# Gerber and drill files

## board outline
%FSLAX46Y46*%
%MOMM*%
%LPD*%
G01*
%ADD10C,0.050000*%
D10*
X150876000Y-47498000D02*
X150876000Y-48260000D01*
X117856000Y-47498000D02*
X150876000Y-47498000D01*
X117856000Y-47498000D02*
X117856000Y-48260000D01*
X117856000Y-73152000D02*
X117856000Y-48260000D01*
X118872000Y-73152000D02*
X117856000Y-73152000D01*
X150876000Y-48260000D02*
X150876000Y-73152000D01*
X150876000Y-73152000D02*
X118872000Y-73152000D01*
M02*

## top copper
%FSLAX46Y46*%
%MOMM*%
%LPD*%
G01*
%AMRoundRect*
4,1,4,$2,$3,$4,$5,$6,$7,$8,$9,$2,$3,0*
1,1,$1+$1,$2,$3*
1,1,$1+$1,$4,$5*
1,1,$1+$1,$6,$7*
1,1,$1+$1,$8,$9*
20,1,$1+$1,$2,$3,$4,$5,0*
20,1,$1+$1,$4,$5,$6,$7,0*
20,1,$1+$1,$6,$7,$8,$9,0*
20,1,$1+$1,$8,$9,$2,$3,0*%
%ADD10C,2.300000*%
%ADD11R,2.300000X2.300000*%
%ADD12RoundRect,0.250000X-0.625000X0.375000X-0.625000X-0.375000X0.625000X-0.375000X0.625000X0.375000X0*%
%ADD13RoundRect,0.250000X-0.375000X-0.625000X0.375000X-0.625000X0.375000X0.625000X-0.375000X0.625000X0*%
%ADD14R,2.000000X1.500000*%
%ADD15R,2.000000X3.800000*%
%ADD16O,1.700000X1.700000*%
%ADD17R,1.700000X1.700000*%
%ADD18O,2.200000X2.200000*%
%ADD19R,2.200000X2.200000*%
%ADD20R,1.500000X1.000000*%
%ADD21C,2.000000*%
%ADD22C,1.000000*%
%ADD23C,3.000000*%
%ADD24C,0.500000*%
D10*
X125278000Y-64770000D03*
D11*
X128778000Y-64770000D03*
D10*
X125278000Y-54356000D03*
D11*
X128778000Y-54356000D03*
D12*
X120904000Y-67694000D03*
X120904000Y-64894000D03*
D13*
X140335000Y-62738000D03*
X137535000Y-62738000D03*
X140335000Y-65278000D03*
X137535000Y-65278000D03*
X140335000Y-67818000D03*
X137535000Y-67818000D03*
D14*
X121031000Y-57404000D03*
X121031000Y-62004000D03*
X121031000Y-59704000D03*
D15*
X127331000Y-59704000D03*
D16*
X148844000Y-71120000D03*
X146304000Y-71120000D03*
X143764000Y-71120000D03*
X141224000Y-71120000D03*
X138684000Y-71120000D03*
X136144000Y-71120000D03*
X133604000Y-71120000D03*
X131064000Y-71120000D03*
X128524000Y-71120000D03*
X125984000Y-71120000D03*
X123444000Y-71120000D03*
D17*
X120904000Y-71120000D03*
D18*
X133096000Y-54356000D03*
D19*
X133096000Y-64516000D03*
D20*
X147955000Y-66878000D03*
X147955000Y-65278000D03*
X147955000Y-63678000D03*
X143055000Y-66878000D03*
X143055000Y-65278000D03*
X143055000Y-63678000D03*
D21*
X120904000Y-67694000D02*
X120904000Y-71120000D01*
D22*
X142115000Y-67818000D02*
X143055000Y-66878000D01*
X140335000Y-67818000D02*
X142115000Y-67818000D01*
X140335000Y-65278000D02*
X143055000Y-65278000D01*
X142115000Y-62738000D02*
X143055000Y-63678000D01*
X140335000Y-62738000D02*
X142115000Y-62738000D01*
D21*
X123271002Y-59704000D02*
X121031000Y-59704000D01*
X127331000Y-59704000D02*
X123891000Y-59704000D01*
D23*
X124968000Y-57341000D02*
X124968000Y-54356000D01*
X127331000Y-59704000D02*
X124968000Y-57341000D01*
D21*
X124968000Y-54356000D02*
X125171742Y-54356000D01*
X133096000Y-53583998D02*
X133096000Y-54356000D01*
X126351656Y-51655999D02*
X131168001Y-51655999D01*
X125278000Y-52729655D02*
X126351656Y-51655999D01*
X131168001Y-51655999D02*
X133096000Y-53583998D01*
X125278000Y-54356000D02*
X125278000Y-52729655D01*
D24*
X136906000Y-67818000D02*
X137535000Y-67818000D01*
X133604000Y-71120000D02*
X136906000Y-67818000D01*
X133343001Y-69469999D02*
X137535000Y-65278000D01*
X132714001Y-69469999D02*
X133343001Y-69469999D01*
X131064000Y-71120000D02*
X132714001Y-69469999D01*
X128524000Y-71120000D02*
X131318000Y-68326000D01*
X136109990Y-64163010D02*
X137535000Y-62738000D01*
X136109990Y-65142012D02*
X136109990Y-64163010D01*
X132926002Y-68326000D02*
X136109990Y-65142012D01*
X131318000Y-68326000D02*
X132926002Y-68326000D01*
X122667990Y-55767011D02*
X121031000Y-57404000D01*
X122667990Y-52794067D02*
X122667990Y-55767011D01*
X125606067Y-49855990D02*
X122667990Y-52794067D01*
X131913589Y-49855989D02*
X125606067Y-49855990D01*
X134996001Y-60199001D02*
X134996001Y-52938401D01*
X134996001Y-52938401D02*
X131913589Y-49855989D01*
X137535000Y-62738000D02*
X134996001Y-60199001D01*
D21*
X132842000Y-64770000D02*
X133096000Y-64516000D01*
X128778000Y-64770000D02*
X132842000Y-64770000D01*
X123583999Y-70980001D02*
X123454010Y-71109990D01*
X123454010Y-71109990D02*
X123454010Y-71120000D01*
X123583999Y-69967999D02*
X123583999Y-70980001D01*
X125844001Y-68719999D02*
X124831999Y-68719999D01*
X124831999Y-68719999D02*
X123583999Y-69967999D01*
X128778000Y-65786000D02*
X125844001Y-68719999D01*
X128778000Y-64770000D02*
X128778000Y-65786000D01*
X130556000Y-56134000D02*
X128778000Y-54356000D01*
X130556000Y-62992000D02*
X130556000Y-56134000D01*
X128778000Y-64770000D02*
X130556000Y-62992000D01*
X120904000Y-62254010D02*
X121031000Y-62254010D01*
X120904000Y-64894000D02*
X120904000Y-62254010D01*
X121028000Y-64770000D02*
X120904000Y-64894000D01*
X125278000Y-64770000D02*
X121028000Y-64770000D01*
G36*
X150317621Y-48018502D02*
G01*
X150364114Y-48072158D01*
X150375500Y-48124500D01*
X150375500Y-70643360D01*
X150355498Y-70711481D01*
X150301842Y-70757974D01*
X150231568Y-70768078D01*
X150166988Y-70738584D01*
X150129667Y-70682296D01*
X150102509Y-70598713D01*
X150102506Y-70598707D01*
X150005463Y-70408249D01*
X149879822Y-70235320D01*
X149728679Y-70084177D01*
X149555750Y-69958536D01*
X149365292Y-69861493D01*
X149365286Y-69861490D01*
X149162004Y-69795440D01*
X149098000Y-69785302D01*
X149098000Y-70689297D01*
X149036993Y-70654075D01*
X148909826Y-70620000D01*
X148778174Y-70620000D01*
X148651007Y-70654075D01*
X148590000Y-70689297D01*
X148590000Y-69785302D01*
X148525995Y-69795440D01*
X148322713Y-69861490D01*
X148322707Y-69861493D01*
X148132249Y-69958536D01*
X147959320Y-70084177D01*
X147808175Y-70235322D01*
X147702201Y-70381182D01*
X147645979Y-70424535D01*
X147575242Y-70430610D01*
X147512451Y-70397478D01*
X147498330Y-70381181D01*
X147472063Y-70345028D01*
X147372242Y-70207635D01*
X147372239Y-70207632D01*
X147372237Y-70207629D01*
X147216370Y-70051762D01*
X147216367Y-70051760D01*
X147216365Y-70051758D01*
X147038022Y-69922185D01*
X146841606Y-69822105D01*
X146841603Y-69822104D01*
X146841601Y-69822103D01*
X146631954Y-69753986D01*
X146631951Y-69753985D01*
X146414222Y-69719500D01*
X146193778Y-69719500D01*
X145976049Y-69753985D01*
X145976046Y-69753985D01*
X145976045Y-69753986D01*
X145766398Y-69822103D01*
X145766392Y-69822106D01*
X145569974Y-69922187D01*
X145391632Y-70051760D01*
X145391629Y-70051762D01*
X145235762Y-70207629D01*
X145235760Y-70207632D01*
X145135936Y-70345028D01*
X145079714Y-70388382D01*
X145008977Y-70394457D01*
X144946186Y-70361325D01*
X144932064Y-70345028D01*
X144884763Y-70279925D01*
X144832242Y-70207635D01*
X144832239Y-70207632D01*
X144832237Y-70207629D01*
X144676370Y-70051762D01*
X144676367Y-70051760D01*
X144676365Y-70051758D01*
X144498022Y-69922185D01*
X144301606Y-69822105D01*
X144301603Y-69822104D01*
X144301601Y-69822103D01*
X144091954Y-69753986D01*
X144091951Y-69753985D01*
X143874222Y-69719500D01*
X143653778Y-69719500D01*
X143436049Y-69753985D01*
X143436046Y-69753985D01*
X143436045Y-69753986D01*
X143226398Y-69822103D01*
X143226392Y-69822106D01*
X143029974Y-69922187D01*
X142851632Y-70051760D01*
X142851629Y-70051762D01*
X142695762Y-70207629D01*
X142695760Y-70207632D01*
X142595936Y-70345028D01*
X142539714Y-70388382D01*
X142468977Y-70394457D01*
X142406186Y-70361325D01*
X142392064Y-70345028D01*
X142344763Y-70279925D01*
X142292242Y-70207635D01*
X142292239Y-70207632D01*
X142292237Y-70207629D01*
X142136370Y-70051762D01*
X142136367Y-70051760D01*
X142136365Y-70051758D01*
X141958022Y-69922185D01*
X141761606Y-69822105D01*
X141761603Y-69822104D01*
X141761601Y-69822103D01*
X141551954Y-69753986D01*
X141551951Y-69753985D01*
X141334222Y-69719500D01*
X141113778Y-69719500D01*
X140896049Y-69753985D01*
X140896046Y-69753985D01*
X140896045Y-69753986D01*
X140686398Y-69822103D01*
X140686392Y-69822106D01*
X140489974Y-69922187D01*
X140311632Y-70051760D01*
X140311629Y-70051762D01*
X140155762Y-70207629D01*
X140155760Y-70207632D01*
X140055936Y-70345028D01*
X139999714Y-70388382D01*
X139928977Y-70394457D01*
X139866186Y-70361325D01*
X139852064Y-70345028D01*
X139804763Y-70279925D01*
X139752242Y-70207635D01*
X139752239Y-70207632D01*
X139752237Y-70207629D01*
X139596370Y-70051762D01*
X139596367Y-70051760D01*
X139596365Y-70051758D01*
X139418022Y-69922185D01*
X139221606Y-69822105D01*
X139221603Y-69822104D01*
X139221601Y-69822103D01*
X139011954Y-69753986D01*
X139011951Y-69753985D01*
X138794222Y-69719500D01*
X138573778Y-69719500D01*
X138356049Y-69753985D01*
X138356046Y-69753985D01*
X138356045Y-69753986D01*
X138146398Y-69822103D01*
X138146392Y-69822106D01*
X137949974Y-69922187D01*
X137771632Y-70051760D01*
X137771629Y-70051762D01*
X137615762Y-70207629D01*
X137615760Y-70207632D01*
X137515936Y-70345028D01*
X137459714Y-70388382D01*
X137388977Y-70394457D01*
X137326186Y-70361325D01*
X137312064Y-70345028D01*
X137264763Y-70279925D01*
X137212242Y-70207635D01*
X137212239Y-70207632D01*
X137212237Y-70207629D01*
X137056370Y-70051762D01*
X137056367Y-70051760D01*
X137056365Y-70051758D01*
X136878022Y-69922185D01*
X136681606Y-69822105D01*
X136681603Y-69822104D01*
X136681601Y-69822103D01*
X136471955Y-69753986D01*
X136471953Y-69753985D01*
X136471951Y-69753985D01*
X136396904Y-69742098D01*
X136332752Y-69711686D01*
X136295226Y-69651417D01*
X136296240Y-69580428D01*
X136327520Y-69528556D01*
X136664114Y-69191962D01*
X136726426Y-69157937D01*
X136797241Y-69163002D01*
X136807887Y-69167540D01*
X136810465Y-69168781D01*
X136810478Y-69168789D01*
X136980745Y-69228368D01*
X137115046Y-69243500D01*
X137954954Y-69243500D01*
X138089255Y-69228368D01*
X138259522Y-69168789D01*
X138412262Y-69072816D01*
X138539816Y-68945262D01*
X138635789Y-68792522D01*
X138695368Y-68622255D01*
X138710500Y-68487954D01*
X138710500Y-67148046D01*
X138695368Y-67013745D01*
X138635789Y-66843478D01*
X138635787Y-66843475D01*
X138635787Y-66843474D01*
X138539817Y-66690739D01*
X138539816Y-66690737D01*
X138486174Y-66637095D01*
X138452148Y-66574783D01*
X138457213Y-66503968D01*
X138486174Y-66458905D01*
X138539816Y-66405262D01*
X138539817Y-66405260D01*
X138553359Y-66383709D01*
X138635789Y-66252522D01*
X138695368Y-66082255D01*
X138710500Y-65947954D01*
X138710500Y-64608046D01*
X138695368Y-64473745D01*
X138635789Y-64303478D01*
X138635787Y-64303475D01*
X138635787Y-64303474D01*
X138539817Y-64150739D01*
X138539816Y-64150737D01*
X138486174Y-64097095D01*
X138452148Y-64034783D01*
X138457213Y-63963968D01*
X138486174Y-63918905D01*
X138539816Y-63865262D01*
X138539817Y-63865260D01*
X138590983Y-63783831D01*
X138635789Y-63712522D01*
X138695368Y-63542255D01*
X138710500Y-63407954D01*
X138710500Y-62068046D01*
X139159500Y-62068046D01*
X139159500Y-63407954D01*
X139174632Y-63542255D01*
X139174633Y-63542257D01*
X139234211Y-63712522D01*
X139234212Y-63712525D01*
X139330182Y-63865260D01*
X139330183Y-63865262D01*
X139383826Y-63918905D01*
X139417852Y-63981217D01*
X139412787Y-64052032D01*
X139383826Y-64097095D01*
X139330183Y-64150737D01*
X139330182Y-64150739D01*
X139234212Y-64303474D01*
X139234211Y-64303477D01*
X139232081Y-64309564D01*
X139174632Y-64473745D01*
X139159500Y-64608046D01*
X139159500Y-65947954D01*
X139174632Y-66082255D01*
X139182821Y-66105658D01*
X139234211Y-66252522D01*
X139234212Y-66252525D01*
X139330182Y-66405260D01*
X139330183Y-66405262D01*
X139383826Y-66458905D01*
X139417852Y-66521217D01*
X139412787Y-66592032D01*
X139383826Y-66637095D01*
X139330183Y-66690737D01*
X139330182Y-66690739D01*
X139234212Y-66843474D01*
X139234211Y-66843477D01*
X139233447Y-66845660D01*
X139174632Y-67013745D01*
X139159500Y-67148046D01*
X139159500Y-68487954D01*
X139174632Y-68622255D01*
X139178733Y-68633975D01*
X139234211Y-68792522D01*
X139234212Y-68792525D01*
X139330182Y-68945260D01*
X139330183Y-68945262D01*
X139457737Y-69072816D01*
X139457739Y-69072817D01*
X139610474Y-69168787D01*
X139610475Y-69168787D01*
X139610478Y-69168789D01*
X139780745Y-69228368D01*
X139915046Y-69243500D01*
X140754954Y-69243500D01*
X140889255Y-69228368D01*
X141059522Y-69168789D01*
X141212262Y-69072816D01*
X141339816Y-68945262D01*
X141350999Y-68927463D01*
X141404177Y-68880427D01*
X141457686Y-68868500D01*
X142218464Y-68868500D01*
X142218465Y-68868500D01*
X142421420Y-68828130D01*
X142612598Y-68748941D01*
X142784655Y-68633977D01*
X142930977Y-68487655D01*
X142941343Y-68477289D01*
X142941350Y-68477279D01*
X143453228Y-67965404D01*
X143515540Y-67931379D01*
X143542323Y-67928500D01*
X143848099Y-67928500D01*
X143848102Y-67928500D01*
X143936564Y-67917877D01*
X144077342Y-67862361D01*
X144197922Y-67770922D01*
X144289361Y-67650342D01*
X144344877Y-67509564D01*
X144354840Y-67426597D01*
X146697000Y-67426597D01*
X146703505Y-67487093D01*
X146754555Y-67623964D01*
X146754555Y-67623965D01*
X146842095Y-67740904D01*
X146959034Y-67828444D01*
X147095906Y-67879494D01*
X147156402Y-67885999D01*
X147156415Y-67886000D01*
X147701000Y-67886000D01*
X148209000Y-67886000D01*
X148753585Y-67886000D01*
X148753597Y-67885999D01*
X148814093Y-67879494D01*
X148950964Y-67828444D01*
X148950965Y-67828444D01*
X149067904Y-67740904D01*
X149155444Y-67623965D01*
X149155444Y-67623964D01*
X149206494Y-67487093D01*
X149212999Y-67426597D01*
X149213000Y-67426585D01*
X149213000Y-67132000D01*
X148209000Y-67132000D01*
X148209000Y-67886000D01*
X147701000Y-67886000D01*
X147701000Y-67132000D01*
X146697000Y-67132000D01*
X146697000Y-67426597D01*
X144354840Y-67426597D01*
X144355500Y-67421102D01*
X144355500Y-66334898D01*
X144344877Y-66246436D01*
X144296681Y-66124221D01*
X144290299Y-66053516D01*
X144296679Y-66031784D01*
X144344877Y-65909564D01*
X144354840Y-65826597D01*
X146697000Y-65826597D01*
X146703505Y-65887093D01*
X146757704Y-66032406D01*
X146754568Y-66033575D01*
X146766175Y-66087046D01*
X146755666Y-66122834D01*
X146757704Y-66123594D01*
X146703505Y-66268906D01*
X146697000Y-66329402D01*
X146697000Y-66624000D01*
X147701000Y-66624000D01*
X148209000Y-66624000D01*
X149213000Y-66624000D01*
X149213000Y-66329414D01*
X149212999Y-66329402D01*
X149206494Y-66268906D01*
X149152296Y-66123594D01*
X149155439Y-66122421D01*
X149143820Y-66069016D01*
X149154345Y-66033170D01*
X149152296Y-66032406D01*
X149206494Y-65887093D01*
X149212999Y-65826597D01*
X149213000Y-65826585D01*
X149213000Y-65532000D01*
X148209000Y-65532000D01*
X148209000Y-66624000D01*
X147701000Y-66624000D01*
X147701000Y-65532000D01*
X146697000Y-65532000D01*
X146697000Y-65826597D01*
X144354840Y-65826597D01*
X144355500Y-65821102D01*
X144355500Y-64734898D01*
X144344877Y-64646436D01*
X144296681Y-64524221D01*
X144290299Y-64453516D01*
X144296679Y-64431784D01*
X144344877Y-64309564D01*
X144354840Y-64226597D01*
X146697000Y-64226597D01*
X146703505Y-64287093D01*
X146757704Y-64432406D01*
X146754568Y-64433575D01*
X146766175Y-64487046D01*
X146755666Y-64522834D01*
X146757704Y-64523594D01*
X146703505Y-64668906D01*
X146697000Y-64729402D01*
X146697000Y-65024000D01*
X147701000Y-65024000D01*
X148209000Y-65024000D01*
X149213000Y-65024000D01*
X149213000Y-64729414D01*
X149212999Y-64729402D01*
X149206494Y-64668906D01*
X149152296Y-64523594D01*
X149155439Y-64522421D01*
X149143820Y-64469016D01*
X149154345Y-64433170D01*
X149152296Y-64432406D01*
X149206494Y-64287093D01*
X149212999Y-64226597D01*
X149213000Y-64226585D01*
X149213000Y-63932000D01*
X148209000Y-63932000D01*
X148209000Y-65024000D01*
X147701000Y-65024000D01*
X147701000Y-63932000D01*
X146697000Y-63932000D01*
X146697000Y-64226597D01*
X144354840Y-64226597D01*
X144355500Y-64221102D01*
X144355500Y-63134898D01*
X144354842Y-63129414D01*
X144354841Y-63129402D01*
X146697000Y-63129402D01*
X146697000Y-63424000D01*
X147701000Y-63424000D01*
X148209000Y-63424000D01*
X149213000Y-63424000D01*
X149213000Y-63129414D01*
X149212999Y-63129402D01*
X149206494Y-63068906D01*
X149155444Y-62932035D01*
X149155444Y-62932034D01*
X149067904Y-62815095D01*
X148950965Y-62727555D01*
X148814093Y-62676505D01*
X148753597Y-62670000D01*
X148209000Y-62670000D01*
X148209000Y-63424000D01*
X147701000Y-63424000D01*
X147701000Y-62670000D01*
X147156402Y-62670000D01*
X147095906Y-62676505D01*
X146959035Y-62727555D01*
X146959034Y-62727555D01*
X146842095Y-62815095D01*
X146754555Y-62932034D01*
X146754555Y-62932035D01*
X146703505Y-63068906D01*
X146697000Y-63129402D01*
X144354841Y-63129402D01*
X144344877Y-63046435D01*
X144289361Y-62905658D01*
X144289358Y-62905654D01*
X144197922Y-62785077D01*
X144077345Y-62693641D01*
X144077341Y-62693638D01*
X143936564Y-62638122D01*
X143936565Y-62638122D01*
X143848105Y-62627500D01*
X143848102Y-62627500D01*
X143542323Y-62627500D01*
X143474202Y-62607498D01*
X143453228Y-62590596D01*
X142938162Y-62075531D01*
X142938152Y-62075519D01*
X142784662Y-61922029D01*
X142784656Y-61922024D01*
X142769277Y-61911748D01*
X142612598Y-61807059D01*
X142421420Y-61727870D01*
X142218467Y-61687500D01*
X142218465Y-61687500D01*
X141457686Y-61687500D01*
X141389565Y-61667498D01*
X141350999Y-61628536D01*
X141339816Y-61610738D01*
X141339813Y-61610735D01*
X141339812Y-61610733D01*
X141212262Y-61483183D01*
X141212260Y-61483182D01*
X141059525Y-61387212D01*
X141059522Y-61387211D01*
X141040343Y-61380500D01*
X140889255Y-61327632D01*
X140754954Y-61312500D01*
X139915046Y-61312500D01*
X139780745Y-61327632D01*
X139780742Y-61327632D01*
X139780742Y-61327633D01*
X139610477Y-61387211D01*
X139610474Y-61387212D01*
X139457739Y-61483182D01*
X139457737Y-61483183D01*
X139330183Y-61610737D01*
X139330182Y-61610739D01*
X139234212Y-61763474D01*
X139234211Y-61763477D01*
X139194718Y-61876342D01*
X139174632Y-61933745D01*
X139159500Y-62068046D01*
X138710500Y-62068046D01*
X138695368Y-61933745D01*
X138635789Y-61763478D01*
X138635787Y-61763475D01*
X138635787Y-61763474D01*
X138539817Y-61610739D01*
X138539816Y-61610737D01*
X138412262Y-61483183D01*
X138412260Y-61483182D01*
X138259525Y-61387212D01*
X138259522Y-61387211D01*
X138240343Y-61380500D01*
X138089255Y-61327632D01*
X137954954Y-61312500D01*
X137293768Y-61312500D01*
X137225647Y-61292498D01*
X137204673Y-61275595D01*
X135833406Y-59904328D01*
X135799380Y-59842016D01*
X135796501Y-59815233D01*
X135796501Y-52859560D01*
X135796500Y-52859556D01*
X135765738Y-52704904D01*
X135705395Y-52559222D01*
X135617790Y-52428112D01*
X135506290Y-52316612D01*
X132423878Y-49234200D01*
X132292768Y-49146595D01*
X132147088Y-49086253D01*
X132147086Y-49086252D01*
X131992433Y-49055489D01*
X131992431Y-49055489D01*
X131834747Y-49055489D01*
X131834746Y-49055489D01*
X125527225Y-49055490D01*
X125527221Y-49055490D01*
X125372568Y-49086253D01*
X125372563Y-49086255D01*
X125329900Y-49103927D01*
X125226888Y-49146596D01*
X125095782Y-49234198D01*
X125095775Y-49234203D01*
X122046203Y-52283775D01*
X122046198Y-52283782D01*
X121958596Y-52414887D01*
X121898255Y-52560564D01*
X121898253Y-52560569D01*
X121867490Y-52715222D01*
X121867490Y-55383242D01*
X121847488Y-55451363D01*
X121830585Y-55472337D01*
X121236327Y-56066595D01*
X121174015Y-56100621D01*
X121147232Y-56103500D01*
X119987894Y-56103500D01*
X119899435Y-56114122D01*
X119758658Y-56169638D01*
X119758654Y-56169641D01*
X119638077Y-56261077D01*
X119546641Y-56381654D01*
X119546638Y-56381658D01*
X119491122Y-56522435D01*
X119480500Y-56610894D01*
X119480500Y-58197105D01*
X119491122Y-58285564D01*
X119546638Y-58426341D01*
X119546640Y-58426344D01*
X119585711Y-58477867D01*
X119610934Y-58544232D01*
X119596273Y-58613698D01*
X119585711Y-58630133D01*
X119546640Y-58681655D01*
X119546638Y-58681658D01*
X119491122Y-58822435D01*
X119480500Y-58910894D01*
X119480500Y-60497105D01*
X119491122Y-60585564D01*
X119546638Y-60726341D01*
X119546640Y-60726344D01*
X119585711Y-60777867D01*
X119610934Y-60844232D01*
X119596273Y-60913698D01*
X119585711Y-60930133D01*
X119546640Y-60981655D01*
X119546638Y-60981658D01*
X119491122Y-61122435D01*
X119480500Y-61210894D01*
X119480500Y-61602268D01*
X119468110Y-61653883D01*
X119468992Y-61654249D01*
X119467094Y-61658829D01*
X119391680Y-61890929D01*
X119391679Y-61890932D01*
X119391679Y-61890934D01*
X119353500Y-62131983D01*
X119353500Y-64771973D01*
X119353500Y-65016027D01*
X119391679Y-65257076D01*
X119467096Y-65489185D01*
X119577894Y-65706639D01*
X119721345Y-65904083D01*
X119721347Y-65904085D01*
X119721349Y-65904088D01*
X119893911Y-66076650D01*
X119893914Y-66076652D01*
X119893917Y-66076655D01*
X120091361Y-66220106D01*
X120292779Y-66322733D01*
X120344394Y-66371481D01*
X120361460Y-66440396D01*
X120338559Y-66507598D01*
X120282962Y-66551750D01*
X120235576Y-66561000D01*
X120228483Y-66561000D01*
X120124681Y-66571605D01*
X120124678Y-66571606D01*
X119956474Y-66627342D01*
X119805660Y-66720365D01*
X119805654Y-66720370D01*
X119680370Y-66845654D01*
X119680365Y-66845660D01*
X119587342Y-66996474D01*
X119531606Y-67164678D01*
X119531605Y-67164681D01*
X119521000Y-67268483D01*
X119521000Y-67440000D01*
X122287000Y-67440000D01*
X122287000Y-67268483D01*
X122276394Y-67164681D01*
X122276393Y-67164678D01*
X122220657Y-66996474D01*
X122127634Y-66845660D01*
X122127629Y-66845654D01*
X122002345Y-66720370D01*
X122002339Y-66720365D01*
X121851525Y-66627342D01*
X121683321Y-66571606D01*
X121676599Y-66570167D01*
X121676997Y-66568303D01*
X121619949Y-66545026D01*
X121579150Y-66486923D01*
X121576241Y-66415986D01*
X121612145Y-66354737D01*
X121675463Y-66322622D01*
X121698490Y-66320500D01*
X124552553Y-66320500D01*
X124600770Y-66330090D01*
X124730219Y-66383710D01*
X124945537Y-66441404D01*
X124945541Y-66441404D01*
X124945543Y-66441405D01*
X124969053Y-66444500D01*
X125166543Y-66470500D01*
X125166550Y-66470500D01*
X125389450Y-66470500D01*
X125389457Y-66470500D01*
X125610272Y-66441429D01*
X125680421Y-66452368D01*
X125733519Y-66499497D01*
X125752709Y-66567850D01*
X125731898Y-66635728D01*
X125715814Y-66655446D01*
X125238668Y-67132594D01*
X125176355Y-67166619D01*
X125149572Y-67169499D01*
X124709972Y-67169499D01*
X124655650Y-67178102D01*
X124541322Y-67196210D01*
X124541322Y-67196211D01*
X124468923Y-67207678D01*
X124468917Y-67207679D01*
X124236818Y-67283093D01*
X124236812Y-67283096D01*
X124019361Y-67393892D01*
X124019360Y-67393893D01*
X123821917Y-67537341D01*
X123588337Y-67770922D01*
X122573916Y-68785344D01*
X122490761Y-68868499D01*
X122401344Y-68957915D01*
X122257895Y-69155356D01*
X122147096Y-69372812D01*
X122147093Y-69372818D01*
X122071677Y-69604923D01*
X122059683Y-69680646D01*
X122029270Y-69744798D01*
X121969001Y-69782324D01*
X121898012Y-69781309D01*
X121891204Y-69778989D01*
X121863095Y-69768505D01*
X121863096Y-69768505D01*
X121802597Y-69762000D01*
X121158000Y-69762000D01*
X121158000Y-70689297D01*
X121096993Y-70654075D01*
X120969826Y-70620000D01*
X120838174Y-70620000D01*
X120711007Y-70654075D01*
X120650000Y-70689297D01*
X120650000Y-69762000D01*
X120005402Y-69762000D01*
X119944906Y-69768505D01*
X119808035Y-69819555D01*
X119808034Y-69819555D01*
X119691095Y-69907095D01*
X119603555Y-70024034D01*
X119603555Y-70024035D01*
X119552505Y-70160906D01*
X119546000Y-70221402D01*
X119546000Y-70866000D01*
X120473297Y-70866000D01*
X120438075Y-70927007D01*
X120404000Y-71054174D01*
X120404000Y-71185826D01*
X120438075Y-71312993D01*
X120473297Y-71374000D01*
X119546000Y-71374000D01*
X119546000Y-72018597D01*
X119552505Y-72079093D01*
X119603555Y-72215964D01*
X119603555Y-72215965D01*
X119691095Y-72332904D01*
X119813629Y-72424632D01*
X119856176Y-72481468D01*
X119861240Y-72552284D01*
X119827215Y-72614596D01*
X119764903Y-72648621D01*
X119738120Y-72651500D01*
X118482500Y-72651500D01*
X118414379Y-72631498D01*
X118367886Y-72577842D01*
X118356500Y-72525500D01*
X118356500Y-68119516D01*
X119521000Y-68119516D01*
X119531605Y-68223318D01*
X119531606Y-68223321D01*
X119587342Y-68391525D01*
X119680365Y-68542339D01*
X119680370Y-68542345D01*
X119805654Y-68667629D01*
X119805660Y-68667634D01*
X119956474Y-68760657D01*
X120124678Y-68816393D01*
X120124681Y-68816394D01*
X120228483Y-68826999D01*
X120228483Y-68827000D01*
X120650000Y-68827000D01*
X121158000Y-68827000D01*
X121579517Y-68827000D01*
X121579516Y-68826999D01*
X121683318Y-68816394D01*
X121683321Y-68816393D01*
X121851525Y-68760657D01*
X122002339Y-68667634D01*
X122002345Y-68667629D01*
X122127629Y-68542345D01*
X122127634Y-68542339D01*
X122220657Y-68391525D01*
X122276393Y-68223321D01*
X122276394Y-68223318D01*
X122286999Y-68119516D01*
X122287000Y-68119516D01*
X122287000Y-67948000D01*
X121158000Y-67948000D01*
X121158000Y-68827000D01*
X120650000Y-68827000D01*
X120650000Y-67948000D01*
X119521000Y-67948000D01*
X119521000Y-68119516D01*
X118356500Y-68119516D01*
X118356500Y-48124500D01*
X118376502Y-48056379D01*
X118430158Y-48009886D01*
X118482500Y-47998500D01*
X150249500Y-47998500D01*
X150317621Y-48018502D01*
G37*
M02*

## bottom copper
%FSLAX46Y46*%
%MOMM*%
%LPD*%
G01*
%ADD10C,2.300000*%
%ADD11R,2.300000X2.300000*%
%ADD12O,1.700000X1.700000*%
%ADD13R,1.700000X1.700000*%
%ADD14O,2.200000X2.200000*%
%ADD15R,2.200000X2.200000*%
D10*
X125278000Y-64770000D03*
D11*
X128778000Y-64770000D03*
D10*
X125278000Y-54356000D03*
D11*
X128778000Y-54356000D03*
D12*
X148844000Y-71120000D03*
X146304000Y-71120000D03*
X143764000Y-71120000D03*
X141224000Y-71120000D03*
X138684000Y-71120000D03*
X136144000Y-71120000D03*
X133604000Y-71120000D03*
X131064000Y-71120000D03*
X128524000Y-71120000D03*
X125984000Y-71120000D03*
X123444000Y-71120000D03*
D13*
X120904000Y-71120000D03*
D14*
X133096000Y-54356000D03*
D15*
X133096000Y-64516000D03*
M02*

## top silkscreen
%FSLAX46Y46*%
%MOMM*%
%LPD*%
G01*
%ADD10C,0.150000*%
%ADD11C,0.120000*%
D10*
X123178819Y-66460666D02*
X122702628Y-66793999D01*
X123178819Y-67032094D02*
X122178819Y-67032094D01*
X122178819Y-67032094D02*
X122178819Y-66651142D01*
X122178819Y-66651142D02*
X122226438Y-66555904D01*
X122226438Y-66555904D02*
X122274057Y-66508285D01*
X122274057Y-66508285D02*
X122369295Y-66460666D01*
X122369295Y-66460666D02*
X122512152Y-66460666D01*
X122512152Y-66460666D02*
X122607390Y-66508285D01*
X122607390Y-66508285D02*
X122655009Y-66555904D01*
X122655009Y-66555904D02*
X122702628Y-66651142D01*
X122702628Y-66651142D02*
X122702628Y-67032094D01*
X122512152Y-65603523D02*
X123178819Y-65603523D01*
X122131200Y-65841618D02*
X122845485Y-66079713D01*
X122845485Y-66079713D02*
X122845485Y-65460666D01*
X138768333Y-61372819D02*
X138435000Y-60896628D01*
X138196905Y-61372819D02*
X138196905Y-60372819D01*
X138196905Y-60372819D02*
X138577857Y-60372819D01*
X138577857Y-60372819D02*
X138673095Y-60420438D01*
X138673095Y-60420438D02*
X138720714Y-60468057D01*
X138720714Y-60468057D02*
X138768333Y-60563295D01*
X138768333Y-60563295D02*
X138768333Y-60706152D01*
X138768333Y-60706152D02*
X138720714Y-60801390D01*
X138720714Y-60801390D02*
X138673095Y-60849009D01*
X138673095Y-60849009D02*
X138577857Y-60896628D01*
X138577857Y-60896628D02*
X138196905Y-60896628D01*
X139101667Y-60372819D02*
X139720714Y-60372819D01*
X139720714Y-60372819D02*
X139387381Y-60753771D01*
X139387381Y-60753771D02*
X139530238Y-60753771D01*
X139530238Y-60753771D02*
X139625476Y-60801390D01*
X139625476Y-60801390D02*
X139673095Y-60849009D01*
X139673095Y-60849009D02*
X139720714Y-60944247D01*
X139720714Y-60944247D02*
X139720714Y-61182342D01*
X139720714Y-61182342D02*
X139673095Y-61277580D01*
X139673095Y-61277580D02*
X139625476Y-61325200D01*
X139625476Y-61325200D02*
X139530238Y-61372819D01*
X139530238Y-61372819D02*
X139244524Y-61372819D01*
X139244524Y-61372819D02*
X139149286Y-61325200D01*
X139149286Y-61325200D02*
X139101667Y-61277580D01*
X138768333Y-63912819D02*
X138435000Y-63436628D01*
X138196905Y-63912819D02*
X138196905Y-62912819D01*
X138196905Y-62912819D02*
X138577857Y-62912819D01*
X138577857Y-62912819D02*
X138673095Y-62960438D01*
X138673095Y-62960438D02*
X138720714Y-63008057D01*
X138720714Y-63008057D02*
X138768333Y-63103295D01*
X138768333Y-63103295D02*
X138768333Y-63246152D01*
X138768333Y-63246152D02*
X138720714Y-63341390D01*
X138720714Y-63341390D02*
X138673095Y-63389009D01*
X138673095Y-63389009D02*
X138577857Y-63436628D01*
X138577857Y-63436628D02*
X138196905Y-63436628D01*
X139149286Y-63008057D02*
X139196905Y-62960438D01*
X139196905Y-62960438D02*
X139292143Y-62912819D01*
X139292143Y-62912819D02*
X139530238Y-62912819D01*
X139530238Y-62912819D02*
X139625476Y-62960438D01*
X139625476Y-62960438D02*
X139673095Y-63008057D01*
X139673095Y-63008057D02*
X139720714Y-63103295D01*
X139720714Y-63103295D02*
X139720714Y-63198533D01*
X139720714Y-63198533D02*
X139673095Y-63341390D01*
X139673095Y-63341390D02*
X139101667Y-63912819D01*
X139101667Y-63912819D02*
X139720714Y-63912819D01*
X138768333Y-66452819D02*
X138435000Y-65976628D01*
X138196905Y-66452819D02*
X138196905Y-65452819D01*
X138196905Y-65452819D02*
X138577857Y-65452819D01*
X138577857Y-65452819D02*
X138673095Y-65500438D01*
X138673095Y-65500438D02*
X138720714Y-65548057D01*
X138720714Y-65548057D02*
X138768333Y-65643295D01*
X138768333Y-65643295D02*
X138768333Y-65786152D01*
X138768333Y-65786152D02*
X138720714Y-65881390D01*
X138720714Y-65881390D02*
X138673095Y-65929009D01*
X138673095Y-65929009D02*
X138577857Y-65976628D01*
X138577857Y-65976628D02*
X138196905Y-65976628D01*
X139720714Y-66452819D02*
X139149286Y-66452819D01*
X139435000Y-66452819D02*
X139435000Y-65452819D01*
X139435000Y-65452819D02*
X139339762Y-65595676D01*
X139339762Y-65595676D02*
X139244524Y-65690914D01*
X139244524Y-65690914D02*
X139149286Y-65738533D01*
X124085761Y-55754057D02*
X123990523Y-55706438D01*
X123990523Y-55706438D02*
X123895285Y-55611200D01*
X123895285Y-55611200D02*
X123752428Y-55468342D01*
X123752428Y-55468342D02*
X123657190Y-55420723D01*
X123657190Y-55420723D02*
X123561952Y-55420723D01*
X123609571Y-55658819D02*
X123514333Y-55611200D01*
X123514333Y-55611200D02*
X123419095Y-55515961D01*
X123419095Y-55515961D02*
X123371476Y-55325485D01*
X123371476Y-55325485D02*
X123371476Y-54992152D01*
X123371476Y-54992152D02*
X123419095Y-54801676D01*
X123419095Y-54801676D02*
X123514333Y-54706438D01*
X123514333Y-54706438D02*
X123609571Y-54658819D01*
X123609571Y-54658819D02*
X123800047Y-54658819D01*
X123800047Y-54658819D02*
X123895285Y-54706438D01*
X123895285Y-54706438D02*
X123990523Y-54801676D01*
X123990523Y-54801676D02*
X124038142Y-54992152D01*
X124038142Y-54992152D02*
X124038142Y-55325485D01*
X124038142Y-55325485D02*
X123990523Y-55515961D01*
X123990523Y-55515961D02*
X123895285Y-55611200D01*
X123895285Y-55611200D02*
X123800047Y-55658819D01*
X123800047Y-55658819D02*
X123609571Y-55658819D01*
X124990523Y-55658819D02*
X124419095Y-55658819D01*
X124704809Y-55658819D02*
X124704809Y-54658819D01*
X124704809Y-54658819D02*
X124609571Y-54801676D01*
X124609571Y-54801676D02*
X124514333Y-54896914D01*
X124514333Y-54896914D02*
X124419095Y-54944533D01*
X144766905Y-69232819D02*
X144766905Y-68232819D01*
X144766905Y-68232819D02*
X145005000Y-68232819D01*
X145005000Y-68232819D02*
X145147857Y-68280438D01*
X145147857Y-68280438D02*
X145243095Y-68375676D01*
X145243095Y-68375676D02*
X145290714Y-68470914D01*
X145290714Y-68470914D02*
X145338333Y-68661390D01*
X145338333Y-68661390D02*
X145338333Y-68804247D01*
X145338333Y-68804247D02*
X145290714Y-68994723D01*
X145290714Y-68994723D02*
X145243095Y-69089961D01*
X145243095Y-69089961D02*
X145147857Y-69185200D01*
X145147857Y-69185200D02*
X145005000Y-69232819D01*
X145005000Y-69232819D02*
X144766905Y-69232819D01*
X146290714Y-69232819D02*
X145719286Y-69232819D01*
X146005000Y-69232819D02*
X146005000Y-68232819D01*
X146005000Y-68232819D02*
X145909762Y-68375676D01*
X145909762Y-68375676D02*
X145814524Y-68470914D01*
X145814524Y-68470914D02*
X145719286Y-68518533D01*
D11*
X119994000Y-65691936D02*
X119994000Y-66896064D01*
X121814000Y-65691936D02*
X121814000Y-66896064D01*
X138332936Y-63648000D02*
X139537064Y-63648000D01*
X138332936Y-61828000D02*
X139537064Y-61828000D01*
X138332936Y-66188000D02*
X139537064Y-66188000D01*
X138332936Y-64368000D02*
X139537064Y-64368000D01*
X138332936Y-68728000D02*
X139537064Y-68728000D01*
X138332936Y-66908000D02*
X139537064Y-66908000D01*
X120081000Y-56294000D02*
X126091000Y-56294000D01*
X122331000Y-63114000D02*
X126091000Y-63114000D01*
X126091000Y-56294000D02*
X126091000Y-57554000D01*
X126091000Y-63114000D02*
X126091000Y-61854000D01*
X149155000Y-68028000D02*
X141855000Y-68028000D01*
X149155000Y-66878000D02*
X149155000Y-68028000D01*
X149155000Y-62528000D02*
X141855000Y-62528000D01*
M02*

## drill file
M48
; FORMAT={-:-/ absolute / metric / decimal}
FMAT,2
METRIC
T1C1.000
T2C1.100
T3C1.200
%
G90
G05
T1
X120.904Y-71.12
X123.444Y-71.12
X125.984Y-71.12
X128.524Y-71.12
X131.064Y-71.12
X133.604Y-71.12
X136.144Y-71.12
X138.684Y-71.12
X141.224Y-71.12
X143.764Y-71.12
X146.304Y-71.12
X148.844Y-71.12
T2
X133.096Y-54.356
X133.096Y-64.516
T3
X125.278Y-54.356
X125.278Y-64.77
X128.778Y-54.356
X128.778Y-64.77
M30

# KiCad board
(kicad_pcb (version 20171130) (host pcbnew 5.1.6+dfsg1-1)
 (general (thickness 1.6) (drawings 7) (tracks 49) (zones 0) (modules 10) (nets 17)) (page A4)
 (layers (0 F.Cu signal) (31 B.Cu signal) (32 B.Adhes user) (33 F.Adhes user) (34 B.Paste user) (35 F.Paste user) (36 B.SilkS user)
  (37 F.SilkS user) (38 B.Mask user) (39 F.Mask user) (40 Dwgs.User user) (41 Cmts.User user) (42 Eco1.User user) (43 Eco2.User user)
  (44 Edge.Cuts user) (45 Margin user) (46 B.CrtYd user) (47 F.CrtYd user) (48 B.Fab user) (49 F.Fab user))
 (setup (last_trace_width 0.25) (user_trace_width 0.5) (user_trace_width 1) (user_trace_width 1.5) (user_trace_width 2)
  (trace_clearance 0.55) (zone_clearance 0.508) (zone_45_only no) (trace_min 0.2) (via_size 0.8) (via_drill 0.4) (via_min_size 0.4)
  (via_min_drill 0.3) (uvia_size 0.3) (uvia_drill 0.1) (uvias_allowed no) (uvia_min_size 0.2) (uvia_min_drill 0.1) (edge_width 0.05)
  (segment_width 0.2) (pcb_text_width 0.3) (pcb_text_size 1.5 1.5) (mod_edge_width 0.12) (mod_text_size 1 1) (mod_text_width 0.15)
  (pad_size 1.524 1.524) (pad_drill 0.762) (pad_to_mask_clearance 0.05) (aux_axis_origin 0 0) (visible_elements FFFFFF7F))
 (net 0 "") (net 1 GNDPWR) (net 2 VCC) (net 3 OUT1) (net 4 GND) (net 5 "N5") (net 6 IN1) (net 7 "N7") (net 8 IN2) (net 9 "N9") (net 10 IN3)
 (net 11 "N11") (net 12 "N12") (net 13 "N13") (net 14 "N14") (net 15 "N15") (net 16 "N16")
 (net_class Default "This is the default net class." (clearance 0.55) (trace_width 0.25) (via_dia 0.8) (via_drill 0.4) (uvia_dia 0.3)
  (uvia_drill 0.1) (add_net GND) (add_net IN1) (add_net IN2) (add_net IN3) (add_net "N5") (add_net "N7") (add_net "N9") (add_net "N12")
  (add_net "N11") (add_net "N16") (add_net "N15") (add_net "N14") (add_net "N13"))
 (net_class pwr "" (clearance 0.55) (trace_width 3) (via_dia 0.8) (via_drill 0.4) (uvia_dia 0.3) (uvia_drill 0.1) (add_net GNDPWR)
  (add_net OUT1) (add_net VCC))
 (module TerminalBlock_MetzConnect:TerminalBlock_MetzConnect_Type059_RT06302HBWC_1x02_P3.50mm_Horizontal (layer B.Cu) (at 128.778 64.77 180)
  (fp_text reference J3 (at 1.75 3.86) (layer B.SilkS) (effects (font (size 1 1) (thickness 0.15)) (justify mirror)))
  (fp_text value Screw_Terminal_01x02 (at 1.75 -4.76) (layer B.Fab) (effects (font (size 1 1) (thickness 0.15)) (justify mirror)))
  (pad 2 thru_hole circle (at 3.5 0 180) (size 2.3 2.3) (drill 1.2) (layers *.Cu *.Mask) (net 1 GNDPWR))
  (pad 1 thru_hole rect (at 0 0 180) (size 2.3 2.3) (drill 1.2) (layers *.Cu *.Mask) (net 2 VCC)))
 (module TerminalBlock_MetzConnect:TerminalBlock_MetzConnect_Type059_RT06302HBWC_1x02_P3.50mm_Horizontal (layer B.Cu)
  (at 128.778 54.356 180)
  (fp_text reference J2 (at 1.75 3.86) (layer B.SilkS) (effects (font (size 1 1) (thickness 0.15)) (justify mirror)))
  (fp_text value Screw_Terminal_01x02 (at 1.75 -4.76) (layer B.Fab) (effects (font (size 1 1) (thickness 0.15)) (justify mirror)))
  (pad 2 thru_hole circle (at 3.5 0 180) (size 2.3 2.3) (drill 1.2) (layers *.Cu *.Mask) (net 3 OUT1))
  (pad 1 thru_hole rect (at 0 0 180) (size 2.3 2.3) (drill 1.2) (layers *.Cu *.Mask) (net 2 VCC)))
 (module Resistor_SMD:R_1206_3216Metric (layer F.Cu) (at 120.904 66.294 270)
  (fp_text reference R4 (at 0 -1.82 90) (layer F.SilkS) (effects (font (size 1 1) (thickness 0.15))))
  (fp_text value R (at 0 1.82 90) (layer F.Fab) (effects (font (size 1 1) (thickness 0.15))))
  (fp_line (start -0.602064 0.91) (end 0.602064 0.91) (layer F.SilkS) (width 0.12))
  (fp_line (start -0.602064 -0.91) (end 0.602064 -0.91) (layer F.SilkS) (width 0.12))
  (pad 2 smd roundrect (at 1.4 0 270) (size 1.25 1.75) (layers F.Cu F.Paste F.Mask) (roundrect_rratio 0.2) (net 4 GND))
  (pad 1 smd roundrect (at -1.4 0 270) (size 1.25 1.75) (layers F.Cu F.Paste F.Mask) (roundrect_rratio 0.2) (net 1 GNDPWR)))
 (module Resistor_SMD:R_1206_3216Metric (layer F.Cu) (at 138.935 62.738)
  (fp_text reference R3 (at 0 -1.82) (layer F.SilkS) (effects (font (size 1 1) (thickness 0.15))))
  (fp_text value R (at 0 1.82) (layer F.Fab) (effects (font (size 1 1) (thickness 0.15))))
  (fp_line (start -0.602064 0.91) (end 0.602064 0.91) (layer F.SilkS) (width 0.12))
  (fp_line (start -0.602064 -0.91) (end 0.602064 -0.91) (layer F.SilkS) (width 0.12))
  (pad 2 smd roundrect (at 1.4 0) (size 1.25 1.75) (layers F.Cu F.Paste F.Mask) (roundrect_rratio 0.2) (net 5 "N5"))
  (pad 1 smd roundrect (at -1.4 0) (size 1.25 1.75) (layers F.Cu F.Paste F.Mask) (roundrect_rratio 0.2) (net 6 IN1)))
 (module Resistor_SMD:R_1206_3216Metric (layer F.Cu) (at 138.935 65.278)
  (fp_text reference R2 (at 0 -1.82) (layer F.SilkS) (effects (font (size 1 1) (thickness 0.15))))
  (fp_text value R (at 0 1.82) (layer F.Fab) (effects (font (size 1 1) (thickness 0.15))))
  (fp_line (start -0.602064 0.91) (end 0.602064 0.91) (layer F.SilkS) (width 0.12))
  (fp_line (start -0.602064 -0.91) (end 0.602064 -0.91) (layer F.SilkS) (width 0.12))
  (pad 2 smd roundrect (at 1.4 0) (size 1.25 1.75) (layers F.Cu F.Paste F.Mask) (roundrect_rratio 0.2) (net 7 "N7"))
  (pad 1 smd roundrect (at -1.4 0) (size 1.25 1.75) (layers F.Cu F.Paste F.Mask) (roundrect_rratio 0.2) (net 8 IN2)))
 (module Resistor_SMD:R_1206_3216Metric (layer F.Cu) (at 138.935 67.818)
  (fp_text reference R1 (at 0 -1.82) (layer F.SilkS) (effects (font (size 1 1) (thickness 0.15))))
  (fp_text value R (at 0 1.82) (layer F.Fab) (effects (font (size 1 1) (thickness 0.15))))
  (fp_line (start -0.602064 0.91) (end 0.602064 0.91) (layer F.SilkS) (width 0.12))
  (fp_line (start -0.602064 -0.91) (end 0.602064 -0.91) (layer F.SilkS) (width 0.12))
  (pad 2 smd roundrect (at 1.4 0) (size 1.25 1.75) (layers F.Cu F.Paste F.Mask) (roundrect_rratio 0.2) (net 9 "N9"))
  (pad 1 smd roundrect (at -1.4 0) (size 1.25 1.75) (layers F.Cu F.Paste F.Mask) (roundrect_rratio 0.2) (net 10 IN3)))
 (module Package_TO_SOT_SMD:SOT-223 (layer F.Cu) (at 124.181 59.704)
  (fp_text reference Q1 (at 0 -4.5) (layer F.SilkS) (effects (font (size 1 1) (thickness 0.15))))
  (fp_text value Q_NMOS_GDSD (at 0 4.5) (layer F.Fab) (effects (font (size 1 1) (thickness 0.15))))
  (fp_line (start -4.1 -3.41) (end 1.91 -3.41) (layer F.SilkS) (width 0.12))
  (fp_line (start -1.85 3.41) (end 1.91 3.41) (layer F.SilkS) (width 0.12))
  (fp_line (start 1.91 -3.41) (end 1.91 -2.15) (layer F.SilkS) (width 0.12))
  (fp_line (start 1.91 3.41) (end 1.91 2.15) (layer F.SilkS) (width 0.12))
  (pad 1 smd rect (at -3.15 -2.3) (size 2 1.5) (layers F.Cu F.Paste F.Mask) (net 6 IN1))
  (pad 3 smd rect (at -3.15 2.3) (size 2 1.5) (layers F.Cu F.Paste F.Mask) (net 1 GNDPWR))
  (pad 2 smd rect (at -3.15 0) (size 2 1.5) (layers F.Cu F.Paste F.Mask) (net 3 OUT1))
  (pad 4 smd rect (at 3.15 0) (size 2 3.8) (layers F.Cu F.Paste F.Mask) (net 3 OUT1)))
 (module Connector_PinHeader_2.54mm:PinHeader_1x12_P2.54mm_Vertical (layer B.Cu) (at 120.904 71.12 270)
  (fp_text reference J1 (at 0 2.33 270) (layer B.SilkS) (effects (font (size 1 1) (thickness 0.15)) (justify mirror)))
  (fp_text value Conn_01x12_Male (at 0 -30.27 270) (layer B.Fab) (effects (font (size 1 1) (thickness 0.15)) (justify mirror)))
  (pad 12 thru_hole oval (at 0 -27.94 270) (size 1.7 1.7) (drill 1) (layers *.Cu *.Mask) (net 4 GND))
  (pad 11 thru_hole oval (at 0 -25.4 270) (size 1.7 1.7) (drill 1) (layers *.Cu *.Mask) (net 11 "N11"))
  (pad 10 thru_hole oval (at 0 -22.86 270) (size 1.7 1.7) (drill 1) (layers *.Cu *.Mask) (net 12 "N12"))
  (pad 9 thru_hole oval (at 0 -20.32 270) (size 1.7 1.7) (drill 1) (layers *.Cu *.Mask) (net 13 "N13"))
  (pad 8 thru_hole oval (at 0 -17.78 270) (size 1.7 1.7) (drill 1) (layers *.Cu *.Mask) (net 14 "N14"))
  (pad 7 thru_hole oval (at 0 -15.24 270) (size 1.7 1.7) (drill 1) (layers *.Cu *.Mask) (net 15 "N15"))
  (pad 6 thru_hole oval (at 0 -12.7 270) (size 1.7 1.7) (drill 1) (layers *.Cu *.Mask) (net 10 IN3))
  (pad 5 thru_hole oval (at 0 -10.16 270) (size 1.7 1.7) (drill 1) (layers *.Cu *.Mask) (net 8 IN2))
  (pad 4 thru_hole oval (at 0 -7.62 270) (size 1.7 1.7) (drill 1) (layers *.Cu *.Mask) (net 6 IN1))
  (pad 3 thru_hole oval (at 0 -5.08 270) (size 1.7 1.7) (drill 1) (layers *.Cu *.Mask) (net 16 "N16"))
  (pad 2 thru_hole oval (at 0 -2.54 270) (size 1.7 1.7) (drill 1) (layers *.Cu *.Mask) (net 2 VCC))
  (pad 1 thru_hole rect (at 0 0 270) (size 1.7 1.7) (drill 1) (layers *.Cu *.Mask) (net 4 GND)))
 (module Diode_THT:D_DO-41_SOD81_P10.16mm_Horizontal (layer B.Cu) (at 133.096 64.516 90)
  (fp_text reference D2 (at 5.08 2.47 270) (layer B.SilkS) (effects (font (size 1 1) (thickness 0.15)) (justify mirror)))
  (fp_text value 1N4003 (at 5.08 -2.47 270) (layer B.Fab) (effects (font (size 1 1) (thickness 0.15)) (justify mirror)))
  (pad 2 thru_hole oval (at 10.16 0 90) (size 2.2 2.2) (drill 1.1) (layers *.Cu *.Mask) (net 3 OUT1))
  (pad 1 thru_hole rect (at 0 0 90) (size 2.2 2.2) (drill 1.1) (layers *.Cu *.Mask) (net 2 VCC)))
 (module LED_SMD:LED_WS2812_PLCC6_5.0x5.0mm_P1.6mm (layer F.Cu) (at 145.505 65.278 180)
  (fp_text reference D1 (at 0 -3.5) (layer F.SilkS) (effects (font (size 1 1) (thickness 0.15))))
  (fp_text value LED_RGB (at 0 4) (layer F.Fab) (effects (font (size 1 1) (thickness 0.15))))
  (fp_line (start -3.65 -2.75) (end 3.65 -2.75) (layer F.SilkS) (width 0.12))
  (fp_line (start -3.65 -1.6) (end -3.65 -2.75) (layer F.SilkS) (width 0.12))
  (fp_line (start -3.65 2.75) (end 3.65 2.75) (layer F.SilkS) (width 0.12))
  (pad 1 smd rect (at -2.45 -1.6 180) (size 1.5 1) (layers F.Cu F.Paste F.Mask) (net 4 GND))
  (pad 2 smd rect (at -2.45 0 180) (size 1.5 1) (layers F.Cu F.Paste F.Mask) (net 4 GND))
  (pad 3 smd rect (at -2.45 1.6 180) (size 1.5 1) (layers F.Cu F.Paste F.Mask) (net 4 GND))
  (pad 6 smd rect (at 2.45 -1.6 180) (size 1.5 1) (layers F.Cu F.Paste F.Mask) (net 9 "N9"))
  (pad 5 smd rect (at 2.45 0 180) (size 1.5 1) (layers F.Cu F.Paste F.Mask) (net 7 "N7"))
  (pad 4 smd rect (at 2.45 1.6 180) (size 1.5 1) (layers F.Cu F.Paste F.Mask) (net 5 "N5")))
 (gr_line (start 150.876 47.498) (end 150.876 48.26) (layer Edge.Cuts) (width 0.05))
 (gr_line (start 117.856 47.498) (end 150.876 47.498) (layer Edge.Cuts) (width 0.05))
 (gr_line (start 117.856 47.498) (end 117.856 48.26) (layer Edge.Cuts) (width 0.05))
 (gr_line (start 117.856 73.152) (end 117.856 48.26) (layer Edge.Cuts) (width 0.05))
 (gr_line (start 118.872 73.152) (end 117.856 73.152) (layer Edge.Cuts) (width 0.05))
 (gr_line (start 150.876 48.26) (end 150.876 73.152) (layer Edge.Cuts) (width 0.05))
 (gr_line (start 150.876 73.152) (end 118.872 73.152) (layer Edge.Cuts) (width 0.05))
 (segment (start 120.904 67.694) (end 120.904 71.12) (width 2) (layer F.Cu) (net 4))
 (segment (start 142.115 67.818) (end 143.055 66.878) (width 1) (layer F.Cu) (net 9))
 (segment (start 140.335 67.818) (end 142.115 67.818) (width 1) (layer F.Cu) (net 9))
 (segment (start 140.335 65.278) (end 143.055 65.278) (width 1) (layer F.Cu) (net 7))
 (segment (start 142.115 62.738) (end 143.055 63.678) (width 1) (layer F.Cu) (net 5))
 (segment (start 140.335 62.738) (end 142.115 62.738) (width 1) (layer F.Cu) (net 5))
 (segment (start 123.271002 59.704) (end 121.031 59.704) (width 2) (layer F.Cu) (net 3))
 (segment (start 127.331 59.704) (end 123.891 59.704) (width 2) (layer F.Cu) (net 3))
 (segment (start 124.968 57.341) (end 124.968 54.356) (width 3) (layer F.Cu) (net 3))
 (segment (start 127.331 59.704) (end 124.968 57.341) (width 3) (layer F.Cu) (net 3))
 (segment (start 124.968 54.356) (end 125.171742 54.356) (width 2) (layer F.Cu) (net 3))
 (segment (start 133.096 53.583998) (end 133.096 54.356) (width 2) (layer F.Cu) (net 3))
 (segment (start 126.351656 51.655999) (end 131.168001 51.655999) (width 2) (layer F.Cu) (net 3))
 (segment (start 125.278 52.729655) (end 126.351656 51.655999) (width 2) (layer F.Cu) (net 3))
 (segment (start 131.168001 51.655999) (end 133.096 53.583998) (width 2) (layer F.Cu) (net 3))
 (segment (start 125.278 54.356) (end 125.278 52.729655) (width 2) (layer F.Cu) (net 3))
 (segment (start 136.906 67.818) (end 137.535 67.818) (width 0.5) (layer F.Cu) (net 10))
 (segment (start 133.604 71.12) (end 136.906 67.818) (width 0.5) (layer F.Cu) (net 10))
 (segment (start 133.343001 69.469999) (end 137.535 65.278) (width 0.5) (layer F.Cu) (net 8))
 (segment (start 132.714001 69.469999) (end 133.343001 69.469999) (width 0.5) (layer F.Cu) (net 8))
 (segment (start 131.064 71.12) (end 132.714001 69.469999) (width 0.5) (layer F.Cu) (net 8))
 (segment (start 128.524 71.12) (end 131.318 68.326) (width 0.5) (layer F.Cu) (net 6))
 (segment (start 136.10999 64.16301) (end 137.535 62.738) (width 0.5) (layer F.Cu) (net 6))
 (segment (start 136.10999 65.142012) (end 136.10999 64.16301) (width 0.5) (layer F.Cu) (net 6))
 (segment (start 132.926002 68.326) (end 136.10999 65.142012) (width 0.5) (layer F.Cu) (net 6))
 (segment (start 131.318 68.326) (end 132.926002 68.326) (width 0.5) (layer F.Cu) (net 6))
 (segment (start 122.66799 55.767011) (end 121.031 57.404) (width 0.5) (layer F.Cu) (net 6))
 (segment (start 122.66799 52.794067) (end 122.66799 55.767011) (width 0.5) (layer F.Cu) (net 6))
 (segment (start 125.606067 49.85599) (end 122.66799 52.794067) (width 0.5) (layer F.Cu) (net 6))
 (segment (start 131.913589 49.855989) (end 125.606067 49.85599) (width 0.5) (layer F.Cu) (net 6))
 (segment (start 134.996001 60.199001) (end 134.996001 52.938401) (width 0.5) (layer F.Cu) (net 6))
 (segment (start 134.996001 52.938401) (end 131.913589 49.855989) (width 0.5) (layer F.Cu) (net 6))
 (segment (start 137.535 62.738) (end 134.996001 60.199001) (width 0.5) (layer F.Cu) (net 6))
 (segment (start 132.842 64.77) (end 133.096 64.516) (width 2) (layer F.Cu) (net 2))
 (segment (start 128.778 64.77) (end 132.842 64.77) (width 2) (layer F.Cu) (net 2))
 (segment (start 123.583999 70.980001) (end 123.45401 71.10999) (width 2) (layer F.Cu) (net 2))
 (segment (start 123.45401 71.10999) (end 123.45401 71.12) (width 2) (layer F.Cu) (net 2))
 (segment (start 123.583999 69.967999) (end 123.583999 70.980001) (width 2) (layer F.Cu) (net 2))
 (segment (start 125.844001 68.719999) (end 124.831999 68.719999) (width 2) (layer F.Cu) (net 2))
 (segment (start 124.831999 68.719999) (end 123.583999 69.967999) (width 2) (layer F.Cu) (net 2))
 (segment (start 128.778 65.786) (end 125.844001 68.719999) (width 2) (layer F.Cu) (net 2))
 (segment (start 128.778 64.77) (end 128.778 65.786) (width 2) (layer F.Cu) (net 2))
 (segment (start 130.556 56.134) (end 128.778 54.356) (width 2) (layer F.Cu) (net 2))
 (segment (start 130.556 62.992) (end 130.556 56.134) (width 2) (layer F.Cu) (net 2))
 (segment (start 128.778 64.77) (end 130.556 62.992) (width 2) (layer F.Cu) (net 2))
 (segment (start 120.904 62.25401) (end 121.031 62.25401) (width 2) (layer F.Cu) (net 1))
 (segment (start 120.904 64.894) (end 120.904 62.25401) (width 2) (layer F.Cu) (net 1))
 (segment (start 121.028 64.77) (end 120.904 64.894) (width 2) (layer F.Cu) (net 1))
 (segment (start 125.278 64.77) (end 121.028 64.77) (width 2) (layer F.Cu) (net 1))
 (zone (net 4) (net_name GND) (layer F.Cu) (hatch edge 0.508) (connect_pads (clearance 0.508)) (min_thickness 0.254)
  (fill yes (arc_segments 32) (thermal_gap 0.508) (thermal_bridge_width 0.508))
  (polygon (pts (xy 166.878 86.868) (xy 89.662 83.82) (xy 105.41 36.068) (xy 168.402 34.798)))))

